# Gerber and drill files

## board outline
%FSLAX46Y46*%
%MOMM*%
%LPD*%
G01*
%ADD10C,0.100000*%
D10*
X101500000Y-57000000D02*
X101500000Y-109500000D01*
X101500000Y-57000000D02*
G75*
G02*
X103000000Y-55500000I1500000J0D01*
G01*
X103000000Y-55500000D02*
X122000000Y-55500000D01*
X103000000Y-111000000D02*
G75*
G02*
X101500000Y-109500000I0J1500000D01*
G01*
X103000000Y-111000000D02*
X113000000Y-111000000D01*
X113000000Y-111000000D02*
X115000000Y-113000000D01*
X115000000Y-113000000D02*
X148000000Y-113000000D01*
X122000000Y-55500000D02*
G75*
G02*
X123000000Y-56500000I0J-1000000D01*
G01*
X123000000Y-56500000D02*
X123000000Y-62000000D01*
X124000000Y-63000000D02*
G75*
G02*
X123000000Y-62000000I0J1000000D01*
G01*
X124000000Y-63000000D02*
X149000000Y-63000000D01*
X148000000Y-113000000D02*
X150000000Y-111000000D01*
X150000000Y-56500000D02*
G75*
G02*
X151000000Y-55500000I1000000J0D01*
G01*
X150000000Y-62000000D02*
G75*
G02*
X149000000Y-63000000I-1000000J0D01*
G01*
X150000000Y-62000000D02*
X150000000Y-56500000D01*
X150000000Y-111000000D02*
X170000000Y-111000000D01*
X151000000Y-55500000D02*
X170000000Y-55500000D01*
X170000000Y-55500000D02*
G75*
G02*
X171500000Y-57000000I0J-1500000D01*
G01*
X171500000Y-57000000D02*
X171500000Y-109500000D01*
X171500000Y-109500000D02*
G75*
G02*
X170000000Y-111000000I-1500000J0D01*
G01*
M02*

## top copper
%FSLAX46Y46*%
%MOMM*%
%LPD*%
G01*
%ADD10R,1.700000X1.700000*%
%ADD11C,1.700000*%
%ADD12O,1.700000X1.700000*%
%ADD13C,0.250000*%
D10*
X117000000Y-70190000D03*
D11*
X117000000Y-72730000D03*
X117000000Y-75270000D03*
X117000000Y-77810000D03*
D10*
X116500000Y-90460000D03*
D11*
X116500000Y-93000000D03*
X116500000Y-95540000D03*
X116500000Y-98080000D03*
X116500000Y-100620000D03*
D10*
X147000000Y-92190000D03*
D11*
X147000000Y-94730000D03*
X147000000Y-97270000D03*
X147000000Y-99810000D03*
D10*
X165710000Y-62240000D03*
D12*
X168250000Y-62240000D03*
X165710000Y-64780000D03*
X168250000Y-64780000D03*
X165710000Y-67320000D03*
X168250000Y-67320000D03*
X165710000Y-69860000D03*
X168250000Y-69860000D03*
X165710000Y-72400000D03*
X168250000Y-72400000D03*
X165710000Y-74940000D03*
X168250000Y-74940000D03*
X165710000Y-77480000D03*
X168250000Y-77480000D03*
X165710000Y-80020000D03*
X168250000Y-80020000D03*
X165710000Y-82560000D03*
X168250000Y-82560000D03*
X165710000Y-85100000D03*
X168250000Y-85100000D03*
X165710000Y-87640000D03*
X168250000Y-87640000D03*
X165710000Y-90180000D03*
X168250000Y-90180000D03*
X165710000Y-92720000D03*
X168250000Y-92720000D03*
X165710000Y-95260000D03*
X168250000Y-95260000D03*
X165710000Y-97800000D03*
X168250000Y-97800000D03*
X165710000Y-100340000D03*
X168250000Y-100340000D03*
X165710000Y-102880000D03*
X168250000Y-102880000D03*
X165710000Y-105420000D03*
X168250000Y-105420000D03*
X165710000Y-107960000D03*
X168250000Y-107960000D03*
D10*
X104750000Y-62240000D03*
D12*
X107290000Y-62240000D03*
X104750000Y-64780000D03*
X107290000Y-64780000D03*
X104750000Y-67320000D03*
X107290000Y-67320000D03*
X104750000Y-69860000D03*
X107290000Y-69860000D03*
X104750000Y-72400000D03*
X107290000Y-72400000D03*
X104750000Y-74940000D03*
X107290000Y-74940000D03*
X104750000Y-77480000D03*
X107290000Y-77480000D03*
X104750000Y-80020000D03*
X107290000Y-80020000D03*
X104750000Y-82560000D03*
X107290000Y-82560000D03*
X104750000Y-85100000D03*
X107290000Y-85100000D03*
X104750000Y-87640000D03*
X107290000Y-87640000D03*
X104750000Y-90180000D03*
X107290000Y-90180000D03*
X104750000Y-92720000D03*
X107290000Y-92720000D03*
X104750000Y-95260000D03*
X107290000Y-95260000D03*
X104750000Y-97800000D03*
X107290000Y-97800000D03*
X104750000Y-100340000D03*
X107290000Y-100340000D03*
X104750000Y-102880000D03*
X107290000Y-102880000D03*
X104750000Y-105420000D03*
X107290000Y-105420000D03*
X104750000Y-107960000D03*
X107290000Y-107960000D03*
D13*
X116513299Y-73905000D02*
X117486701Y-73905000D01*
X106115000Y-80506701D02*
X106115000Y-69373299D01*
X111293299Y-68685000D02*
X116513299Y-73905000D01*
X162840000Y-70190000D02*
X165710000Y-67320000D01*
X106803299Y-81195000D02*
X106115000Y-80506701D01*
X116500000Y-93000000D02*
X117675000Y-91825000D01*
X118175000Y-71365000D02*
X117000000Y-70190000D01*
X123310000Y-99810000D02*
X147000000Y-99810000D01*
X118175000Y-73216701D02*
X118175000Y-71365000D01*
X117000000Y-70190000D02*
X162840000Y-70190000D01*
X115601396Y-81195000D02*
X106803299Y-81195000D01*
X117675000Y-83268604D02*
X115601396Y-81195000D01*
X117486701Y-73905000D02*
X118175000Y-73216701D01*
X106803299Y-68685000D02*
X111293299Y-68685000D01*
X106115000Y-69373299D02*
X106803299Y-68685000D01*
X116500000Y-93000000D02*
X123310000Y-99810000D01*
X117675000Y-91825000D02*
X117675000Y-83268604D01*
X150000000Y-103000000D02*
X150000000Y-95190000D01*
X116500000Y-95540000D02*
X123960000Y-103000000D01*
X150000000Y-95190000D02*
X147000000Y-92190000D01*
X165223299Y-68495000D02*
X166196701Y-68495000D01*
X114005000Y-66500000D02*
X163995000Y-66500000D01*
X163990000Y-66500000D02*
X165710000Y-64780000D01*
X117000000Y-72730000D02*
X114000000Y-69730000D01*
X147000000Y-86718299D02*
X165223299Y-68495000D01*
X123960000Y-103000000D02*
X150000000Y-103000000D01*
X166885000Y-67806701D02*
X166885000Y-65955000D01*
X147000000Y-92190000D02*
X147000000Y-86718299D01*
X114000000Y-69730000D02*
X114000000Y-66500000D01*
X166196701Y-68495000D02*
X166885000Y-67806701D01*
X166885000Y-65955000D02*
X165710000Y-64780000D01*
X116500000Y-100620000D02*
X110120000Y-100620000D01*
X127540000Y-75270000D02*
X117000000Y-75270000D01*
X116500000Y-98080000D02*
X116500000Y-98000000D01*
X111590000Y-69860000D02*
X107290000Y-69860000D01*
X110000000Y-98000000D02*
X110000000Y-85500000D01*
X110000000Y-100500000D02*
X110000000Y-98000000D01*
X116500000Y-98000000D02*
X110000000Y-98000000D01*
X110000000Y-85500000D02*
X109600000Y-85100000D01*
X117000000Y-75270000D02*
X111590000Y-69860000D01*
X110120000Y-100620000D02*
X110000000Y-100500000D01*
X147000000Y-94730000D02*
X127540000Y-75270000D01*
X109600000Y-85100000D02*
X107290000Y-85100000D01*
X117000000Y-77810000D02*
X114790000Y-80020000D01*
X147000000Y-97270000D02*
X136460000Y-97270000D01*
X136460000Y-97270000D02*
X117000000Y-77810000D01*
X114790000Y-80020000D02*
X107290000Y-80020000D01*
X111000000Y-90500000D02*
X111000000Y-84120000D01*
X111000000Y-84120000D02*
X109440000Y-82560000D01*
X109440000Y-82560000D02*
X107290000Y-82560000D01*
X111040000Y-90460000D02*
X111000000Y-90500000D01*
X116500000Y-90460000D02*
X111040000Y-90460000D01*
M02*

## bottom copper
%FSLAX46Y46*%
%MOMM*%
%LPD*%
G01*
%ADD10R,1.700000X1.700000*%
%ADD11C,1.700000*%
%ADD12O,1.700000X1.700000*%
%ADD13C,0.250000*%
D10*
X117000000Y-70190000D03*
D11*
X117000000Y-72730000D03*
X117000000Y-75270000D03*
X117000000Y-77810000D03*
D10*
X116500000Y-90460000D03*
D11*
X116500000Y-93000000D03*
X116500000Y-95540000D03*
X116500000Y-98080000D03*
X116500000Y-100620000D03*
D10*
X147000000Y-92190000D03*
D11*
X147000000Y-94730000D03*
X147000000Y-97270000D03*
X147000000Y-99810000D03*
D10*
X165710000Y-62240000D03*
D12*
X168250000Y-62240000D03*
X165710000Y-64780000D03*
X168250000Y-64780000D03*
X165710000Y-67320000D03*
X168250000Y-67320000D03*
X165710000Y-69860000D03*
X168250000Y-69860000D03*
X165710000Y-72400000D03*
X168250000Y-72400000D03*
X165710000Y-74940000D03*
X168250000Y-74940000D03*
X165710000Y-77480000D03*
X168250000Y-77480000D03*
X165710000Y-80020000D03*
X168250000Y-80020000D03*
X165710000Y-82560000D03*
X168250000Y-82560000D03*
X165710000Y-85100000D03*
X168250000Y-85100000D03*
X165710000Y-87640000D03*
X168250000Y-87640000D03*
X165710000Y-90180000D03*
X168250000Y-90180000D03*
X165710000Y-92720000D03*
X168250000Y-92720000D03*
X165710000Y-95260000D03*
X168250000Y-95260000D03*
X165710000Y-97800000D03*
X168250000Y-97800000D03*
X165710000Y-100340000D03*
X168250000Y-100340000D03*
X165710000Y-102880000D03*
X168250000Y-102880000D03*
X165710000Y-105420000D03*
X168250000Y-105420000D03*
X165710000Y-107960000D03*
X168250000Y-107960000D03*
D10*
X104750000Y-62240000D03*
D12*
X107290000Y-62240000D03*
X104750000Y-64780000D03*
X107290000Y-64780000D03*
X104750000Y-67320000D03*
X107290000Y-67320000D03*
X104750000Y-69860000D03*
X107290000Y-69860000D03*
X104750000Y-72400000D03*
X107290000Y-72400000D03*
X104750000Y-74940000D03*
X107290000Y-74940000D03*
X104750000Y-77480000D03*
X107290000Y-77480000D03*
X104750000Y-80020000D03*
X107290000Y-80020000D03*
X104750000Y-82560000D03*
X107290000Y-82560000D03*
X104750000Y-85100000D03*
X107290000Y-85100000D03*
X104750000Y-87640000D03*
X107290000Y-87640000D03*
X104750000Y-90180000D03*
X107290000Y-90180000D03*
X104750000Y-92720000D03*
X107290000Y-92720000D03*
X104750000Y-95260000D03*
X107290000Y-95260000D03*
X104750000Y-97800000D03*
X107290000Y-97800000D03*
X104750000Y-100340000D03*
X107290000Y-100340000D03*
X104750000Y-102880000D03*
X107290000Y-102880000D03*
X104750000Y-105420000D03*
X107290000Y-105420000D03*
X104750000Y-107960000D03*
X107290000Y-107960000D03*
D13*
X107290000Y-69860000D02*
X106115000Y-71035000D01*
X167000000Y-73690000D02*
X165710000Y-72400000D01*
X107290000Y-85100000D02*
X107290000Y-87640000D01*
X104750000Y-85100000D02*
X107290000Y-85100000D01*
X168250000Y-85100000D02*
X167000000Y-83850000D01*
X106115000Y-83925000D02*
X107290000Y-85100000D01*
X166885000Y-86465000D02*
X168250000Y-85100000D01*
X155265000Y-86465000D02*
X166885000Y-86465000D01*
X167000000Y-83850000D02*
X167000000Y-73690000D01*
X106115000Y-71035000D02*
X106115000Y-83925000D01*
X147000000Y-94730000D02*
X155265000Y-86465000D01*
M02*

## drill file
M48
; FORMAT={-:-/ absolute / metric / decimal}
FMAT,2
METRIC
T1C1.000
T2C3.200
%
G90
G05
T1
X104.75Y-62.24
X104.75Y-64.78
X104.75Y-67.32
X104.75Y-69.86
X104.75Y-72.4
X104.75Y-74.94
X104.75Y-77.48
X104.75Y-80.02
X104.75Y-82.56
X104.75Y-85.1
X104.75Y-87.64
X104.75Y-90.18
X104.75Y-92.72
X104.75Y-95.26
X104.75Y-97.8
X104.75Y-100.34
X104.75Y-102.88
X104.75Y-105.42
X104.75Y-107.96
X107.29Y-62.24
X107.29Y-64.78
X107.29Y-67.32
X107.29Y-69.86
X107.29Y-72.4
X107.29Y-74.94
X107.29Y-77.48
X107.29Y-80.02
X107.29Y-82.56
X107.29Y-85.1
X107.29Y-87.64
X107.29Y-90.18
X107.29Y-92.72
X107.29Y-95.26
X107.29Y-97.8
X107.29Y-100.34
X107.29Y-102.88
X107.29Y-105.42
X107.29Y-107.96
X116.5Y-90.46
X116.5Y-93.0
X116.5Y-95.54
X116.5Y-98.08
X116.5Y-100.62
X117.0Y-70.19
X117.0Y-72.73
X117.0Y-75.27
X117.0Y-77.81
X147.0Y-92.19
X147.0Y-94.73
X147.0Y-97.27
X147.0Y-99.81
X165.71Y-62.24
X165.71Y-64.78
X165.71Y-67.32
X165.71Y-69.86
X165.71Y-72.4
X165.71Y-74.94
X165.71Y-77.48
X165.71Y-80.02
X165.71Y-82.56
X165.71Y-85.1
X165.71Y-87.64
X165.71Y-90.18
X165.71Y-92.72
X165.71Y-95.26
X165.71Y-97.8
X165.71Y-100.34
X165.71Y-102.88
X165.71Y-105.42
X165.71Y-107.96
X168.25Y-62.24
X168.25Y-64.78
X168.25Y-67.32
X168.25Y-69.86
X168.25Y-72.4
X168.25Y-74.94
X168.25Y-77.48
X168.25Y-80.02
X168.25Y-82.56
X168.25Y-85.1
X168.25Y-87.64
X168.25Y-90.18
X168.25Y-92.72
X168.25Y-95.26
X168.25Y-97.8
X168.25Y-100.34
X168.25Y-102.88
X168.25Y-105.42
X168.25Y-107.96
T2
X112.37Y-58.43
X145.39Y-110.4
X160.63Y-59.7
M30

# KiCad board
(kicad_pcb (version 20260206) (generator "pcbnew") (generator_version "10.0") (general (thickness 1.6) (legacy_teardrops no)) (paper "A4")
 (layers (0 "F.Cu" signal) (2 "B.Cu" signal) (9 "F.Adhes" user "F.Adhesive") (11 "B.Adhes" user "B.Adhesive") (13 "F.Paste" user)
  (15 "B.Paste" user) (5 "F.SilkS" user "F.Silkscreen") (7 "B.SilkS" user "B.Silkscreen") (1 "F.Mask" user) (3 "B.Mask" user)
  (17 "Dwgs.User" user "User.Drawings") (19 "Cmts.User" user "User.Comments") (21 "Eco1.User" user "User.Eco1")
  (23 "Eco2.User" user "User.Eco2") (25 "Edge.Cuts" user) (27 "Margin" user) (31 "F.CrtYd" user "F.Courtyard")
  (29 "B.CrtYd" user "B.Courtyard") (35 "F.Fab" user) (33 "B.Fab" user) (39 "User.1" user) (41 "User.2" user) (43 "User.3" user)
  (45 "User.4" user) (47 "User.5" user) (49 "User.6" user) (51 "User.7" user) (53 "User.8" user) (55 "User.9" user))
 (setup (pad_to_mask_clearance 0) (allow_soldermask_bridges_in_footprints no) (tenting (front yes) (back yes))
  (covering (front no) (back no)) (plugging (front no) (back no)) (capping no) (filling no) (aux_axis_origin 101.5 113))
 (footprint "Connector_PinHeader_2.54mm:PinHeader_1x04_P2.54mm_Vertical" (layer "F.Cu") (at 117 70.19)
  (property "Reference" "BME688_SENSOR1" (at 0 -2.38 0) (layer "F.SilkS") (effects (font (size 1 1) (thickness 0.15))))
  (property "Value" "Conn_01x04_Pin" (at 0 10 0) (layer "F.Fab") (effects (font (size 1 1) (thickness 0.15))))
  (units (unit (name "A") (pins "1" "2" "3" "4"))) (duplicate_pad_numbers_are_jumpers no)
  (pad "1" thru_hole rect (at 0 0) (size 1.7 1.7) (drill 1) (layers "*.Cu" "*.Mask") (remove_unused_layers no) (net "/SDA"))
  (pad "2" thru_hole circle (at 0 2.54) (size 1.7 1.7) (drill 1) (layers "*.Cu" "*.Mask") (remove_unused_layers no) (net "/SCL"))
  (pad "3" thru_hole circle (at 0 5.08) (size 1.7 1.7) (drill 1) (layers "*.Cu" "*.Mask") (remove_unused_layers no) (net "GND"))
  (pad "4" thru_hole circle (at 0 7.62) (size 1.7 1.7) (drill 1) (layers "*.Cu" "*.Mask") (remove_unused_layers no) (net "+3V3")))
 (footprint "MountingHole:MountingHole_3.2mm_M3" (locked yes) (layer "F.Cu") (at 160.63 59.7)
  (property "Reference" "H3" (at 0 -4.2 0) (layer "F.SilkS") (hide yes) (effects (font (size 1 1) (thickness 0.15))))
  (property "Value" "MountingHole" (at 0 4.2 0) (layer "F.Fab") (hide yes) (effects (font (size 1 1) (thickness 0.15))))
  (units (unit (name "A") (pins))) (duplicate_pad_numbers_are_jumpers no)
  (pad "" np_thru_hole circle (at 0 0) (size 3.2 3.2) (drill 3.2) (layers "*.Cu" "*.Mask")))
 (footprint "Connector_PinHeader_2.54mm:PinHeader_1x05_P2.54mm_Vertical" (layer "F.Cu") (at 116.5 90.46)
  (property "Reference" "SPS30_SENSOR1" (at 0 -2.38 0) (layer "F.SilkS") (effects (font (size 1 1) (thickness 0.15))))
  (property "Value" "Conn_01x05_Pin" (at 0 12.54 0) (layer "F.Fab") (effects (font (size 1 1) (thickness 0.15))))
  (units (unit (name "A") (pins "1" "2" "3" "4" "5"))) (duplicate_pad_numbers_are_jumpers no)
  (pad "1" thru_hole rect (at 0 0) (size 1.7 1.7) (drill 1) (layers "*.Cu" "*.Mask") (remove_unused_layers no) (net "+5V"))
  (pad "2" thru_hole circle (at 0 2.54) (size 1.7 1.7) (drill 1) (layers "*.Cu" "*.Mask") (remove_unused_layers no) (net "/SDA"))
  (pad "3" thru_hole circle (at 0 5.08) (size 1.7 1.7) (drill 1) (layers "*.Cu" "*.Mask") (remove_unused_layers no) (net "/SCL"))
  (pad "4" thru_hole circle (at 0 7.62) (size 1.7 1.7) (drill 1) (layers "*.Cu" "*.Mask") (remove_unused_layers no) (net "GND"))
  (pad "5" thru_hole circle (at 0 10.16) (size 1.7 1.7) (drill 1) (layers "*.Cu" "*.Mask") (remove_unused_layers no) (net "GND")))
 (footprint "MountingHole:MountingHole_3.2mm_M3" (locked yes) (layer "F.Cu") (at 145.39 110.4)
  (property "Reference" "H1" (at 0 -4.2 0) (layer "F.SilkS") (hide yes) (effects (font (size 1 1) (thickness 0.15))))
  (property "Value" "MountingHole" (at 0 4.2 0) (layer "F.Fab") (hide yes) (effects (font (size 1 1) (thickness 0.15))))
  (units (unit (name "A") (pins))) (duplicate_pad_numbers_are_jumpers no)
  (pad "" np_thru_hole circle (at 0 0) (size 3.2 3.2) (drill 3.2) (layers "*.Cu" "*.Mask")))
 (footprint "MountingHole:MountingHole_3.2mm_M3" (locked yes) (layer "F.Cu") (at 112.37 58.43)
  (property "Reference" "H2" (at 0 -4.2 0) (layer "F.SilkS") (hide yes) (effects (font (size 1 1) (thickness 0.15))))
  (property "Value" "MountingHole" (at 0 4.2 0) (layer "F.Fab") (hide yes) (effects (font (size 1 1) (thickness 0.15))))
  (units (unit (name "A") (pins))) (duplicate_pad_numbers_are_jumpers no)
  (pad "" np_thru_hole circle (at 0 0) (size 3.2 3.2) (drill 3.2) (layers "*.Cu" "*.Mask")))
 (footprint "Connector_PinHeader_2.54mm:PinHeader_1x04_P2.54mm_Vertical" (layer "F.Cu") (at 147 92.19)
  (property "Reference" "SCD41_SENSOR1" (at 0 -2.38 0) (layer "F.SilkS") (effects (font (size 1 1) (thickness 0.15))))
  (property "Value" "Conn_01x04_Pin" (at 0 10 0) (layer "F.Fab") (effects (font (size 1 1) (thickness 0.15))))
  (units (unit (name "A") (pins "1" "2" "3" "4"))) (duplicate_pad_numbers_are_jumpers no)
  (pad "1" thru_hole rect (at 0 0) (size 1.7 1.7) (drill 1) (layers "*.Cu" "*.Mask") (remove_unused_layers no) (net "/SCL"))
  (pad "2" thru_hole circle (at 0 2.54) (size 1.7 1.7) (drill 1) (layers "*.Cu" "*.Mask") (remove_unused_layers no) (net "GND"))
  (pad "3" thru_hole circle (at 0 5.08) (size 1.7 1.7) (drill 1) (layers "*.Cu" "*.Mask") (remove_unused_layers no) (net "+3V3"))
  (pad "4" thru_hole circle (at 0 7.62) (size 1.7 1.7) (drill 1) (layers "*.Cu" "*.Mask") (remove_unused_layers no) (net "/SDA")))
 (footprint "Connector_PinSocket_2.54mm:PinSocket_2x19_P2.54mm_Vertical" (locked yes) (layer "B.Cu") (at 165.71 62.24 180)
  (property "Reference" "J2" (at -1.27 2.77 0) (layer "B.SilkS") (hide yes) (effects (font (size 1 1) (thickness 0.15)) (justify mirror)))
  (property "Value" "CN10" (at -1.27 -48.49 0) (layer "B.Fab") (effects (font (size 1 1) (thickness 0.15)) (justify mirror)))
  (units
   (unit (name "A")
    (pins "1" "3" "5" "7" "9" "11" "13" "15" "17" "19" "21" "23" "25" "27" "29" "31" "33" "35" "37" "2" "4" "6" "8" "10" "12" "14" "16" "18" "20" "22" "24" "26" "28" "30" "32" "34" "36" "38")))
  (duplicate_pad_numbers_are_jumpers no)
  (pad "1" thru_hole rect (at 0 0 180) (size 1.7 1.7) (drill 1) (layers "*.Cu" "*.Mask") (remove_unused_layers no)
   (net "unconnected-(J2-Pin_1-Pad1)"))
  (pad "2" thru_hole oval (at -2.54 0 180) (size 1.7 1.7) (drill 1) (layers "*.Cu" "*.Mask") (remove_unused_layers no)
   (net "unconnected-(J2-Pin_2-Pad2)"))
  (pad "3" thru_hole oval (at 0 -2.54 180) (size 1.7 1.7) (drill 1) (layers "*.Cu" "*.Mask") (remove_unused_layers no) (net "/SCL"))
  (pad "4" thru_hole oval (at -2.54 -2.54 180) (size 1.7 1.7) (drill 1) (layers "*.Cu" "*.Mask") (remove_unused_layers no)
   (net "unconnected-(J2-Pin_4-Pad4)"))
  (pad "5" thru_hole oval (at 0 -5.08 180) (size 1.7 1.7) (drill 1) (layers "*.Cu" "*.Mask") (remove_unused_layers no) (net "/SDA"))
  (pad "6" thru_hole oval (at -2.54 -5.08 180) (size 1.7 1.7) (drill 1) (layers "*.Cu" "*.Mask") (remove_unused_layers no)
   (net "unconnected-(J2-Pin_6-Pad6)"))
  (pad "7" thru_hole oval (at 0 -7.62 180) (size 1.7 1.7) (drill 1) (layers "*.Cu" "*.Mask") (remove_unused_layers no) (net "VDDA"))
  (pad "8" thru_hole oval (at -2.54 -7.62 180) (size 1.7 1.7) (drill 1) (layers "*.Cu" "*.Mask") (remove_unused_layers no)
   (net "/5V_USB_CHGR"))
  (pad "9" thru_hole oval (at 0 -10.16 180) (size 1.7 1.7) (drill 1) (layers "*.Cu" "*.Mask") (remove_unused_layers no) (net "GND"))
  (pad "10" thru_hole oval (at -2.54 -10.16 180) (size 1.7 1.7) (drill 1) (layers "*.Cu" "*.Mask") (remove_unused_layers no)
   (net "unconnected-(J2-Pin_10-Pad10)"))
  (pad "11" thru_hole oval (at 0 -12.7 180) (size 1.7 1.7) (drill 1) (layers "*.Cu" "*.Mask") (remove_unused_layers no)
   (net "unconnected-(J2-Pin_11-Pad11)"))
  (pad "12" thru_hole oval (at -2.54 -12.7 180) (size 1.7 1.7) (drill 1) (layers "*.Cu" "*.Mask") (remove_unused_layers no)
   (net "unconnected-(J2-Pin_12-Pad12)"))
  (pad "13" thru_hole oval (at 0 -15.24 180) (size 1.7 1.7) (drill 1) (layers "*.Cu" "*.Mask") (remove_unused_layers no)
   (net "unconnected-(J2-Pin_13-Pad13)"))
  (pad "14" thru_hole oval (at -2.54 -15.24 180) (size 1.7 1.7) (drill 1) (layers "*.Cu" "*.Mask") (remove_unused_layers no)
   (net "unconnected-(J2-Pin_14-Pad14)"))
  (pad "15" thru_hole oval (at 0 -17.78 180) (size 1.7 1.7) (drill 1) (layers "*.Cu" "*.Mask") (remove_unused_layers no)
   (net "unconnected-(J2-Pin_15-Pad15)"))
  (pad "16" thru_hole oval (at -2.54 -17.78 180) (size 1.7 1.7) (drill 1) (layers "*.Cu" "*.Mask") (remove_unused_layers no)
   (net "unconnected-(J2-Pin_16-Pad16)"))
  (pad "17" thru_hole oval (at 0 -20.32 180) (size 1.7 1.7) (drill 1) (layers "*.Cu" "*.Mask") (remove_unused_layers no)
   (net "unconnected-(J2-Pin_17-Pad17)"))
  (pad "18" thru_hole oval (at -2.54 -20.32 180) (size 1.7 1.7) (drill 1) (layers "*.Cu" "*.Mask") (remove_unused_layers no)
   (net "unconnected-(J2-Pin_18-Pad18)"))
  (pad "19" thru_hole oval (at 0 -22.86 180) (size 1.7 1.7) (drill 1) (layers "*.Cu" "*.Mask") (remove_unused_layers no)
   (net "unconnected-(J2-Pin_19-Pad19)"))
  (pad "20" thru_hole oval (at -2.54 -22.86 180) (size 1.7 1.7) (drill 1) (layers "*.Cu" "*.Mask") (remove_unused_layers no) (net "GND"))
  (pad "21" thru_hole oval (at 0 -25.4 180) (size 1.7 1.7) (drill 1) (layers "*.Cu" "*.Mask") (remove_unused_layers no)
   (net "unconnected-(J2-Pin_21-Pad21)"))
  (pad "22" thru_hole oval (at -2.54 -25.4 180) (size 1.7 1.7) (drill 1) (layers "*.Cu" "*.Mask") (remove_unused_layers no)
   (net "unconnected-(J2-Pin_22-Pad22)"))
  (pad "23" thru_hole oval (at 0 -27.94 180) (size 1.7 1.7) (drill 1) (layers "*.Cu" "*.Mask") (remove_unused_layers no)
   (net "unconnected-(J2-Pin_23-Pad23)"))
  (pad "24" thru_hole oval (at -2.54 -27.94 180) (size 1.7 1.7) (drill 1) (layers "*.Cu" "*.Mask") (remove_unused_layers no)
   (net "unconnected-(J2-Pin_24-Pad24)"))
  (pad "25" thru_hole oval (at 0 -30.48 180) (size 1.7 1.7) (drill 1) (layers "*.Cu" "*.Mask") (remove_unused_layers no)
   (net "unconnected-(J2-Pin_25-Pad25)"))
  (pad "26" thru_hole oval (at -2.54 -30.48 180) (size 1.7 1.7) (drill 1) (layers "*.Cu" "*.Mask") (remove_unused_layers no)
   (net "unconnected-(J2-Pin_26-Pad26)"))
  (pad "27" thru_hole oval (at 0 -33.02 180) (size 1.7 1.7) (drill 1) (layers "*.Cu" "*.Mask") (remove_unused_layers no)
   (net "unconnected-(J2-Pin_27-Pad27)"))
  (pad "28" thru_hole oval (at -2.54 -33.02 180) (size 1.7 1.7) (drill 1) (layers "*.Cu" "*.Mask") (remove_unused_layers no)
   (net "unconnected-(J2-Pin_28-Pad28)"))
  (pad "29" thru_hole oval (at 0 -35.56 180) (size 1.7 1.7) (drill 1) (layers "*.Cu" "*.Mask") (remove_unused_layers no)
   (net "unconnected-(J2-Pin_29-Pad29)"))
  (pad "30" thru_hole oval (at -2.54 -35.56 180) (size 1.7 1.7) (drill 1) (layers "*.Cu" "*.Mask") (remove_unused_layers no)
   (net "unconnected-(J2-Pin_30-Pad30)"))
  (pad "31" thru_hole oval (at 0 -38.1 180) (size 1.7 1.7) (drill 1) (layers "*.Cu" "*.Mask") (remove_unused_layers no)
   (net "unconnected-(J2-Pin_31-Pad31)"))
  (pad "32" thru_hole oval (at -2.54 -38.1 180) (size 1.7 1.7) (drill 1) (layers "*.Cu" "*.Mask") (remove_unused_layers no) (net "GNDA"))
  (pad "33" thru_hole oval (at 0 -40.64 180) (size 1.7 1.7) (drill 1) (layers "*.Cu" "*.Mask") (remove_unused_layers no)
   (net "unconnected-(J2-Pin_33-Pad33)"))
  (pad "34" thru_hole oval (at -2.54 -40.64 180) (size 1.7 1.7) (drill 1) (layers "*.Cu" "*.Mask") (remove_unused_layers no)
   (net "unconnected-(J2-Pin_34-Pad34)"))
  (pad "35" thru_hole oval (at 0 -43.18 180) (size 1.7 1.7) (drill 1) (layers "*.Cu" "*.Mask") (remove_unused_layers no)
   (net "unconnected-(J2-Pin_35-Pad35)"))
  (pad "36" thru_hole oval (at -2.54 -43.18 180) (size 1.7 1.7) (drill 1) (layers "*.Cu" "*.Mask") (remove_unused_layers no)
   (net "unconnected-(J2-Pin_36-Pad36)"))
  (pad "37" thru_hole oval (at 0 -45.72 180) (size 1.7 1.7) (drill 1) (layers "*.Cu" "*.Mask") (remove_unused_layers no)
   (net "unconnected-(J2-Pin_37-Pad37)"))
  (pad "38" thru_hole oval (at -2.54 -45.72 180) (size 1.7 1.7) (drill 1) (layers "*.Cu" "*.Mask") (remove_unused_layers no)
   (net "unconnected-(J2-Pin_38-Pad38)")))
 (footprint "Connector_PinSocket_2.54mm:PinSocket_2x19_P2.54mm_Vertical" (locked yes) (layer "B.Cu") (at 104.75 62.24 180)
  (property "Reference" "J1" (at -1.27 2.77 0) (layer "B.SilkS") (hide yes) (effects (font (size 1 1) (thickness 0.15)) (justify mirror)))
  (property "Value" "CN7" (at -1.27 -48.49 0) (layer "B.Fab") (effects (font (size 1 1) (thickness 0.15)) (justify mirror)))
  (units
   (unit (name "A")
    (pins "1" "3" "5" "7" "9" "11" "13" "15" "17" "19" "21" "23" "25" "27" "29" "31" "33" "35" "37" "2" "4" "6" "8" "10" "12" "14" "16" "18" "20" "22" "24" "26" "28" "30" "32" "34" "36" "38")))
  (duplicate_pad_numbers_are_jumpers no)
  (pad "1" thru_hole rect (at 0 0 180) (size 1.7 1.7) (drill 1) (layers "*.Cu" "*.Mask") (remove_unused_layers no)
   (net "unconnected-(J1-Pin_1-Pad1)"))
  (pad "2" thru_hole oval (at -2.54 0 180) (size 1.7 1.7) (drill 1) (layers "*.Cu" "*.Mask") (remove_unused_layers no)
   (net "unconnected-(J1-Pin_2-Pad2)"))
  (pad "3" thru_hole oval (at 0 -2.54 180) (size 1.7 1.7) (drill 1) (layers "*.Cu" "*.Mask") (remove_unused_layers no)
   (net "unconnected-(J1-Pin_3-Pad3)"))
  (pad "4" thru_hole oval (at -2.54 -2.54 180) (size 1.7 1.7) (drill 1) (layers "*.Cu" "*.Mask") (remove_unused_layers no)
   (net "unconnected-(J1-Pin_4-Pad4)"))
  (pad "5" thru_hole oval (at 0 -5.08 180) (size 1.7 1.7) (drill 1) (layers "*.Cu" "*.Mask") (remove_unused_layers no) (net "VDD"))
  (pad "6" thru_hole oval (at -2.54 -5.08 180) (size 1.7 1.7) (drill 1) (layers "*.Cu" "*.Mask") (remove_unused_layers no) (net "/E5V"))
  (pad "7" thru_hole oval (at 0 -7.62 180) (size 1.7 1.7) (drill 1) (layers "*.Cu" "*.Mask") (remove_unused_layers no)
   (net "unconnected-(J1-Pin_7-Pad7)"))
  (pad "8" thru_hole oval (at -2.54 -7.62 180) (size 1.7 1.7) (drill 1) (layers "*.Cu" "*.Mask") (remove_unused_layers no) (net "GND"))
  (pad "9" thru_hole oval (at 0 -10.16 180) (size 1.7 1.7) (drill 1) (layers "*.Cu" "*.Mask") (remove_unused_layers no)
   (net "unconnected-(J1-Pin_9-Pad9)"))
  (pad "10" thru_hole oval (at -2.54 -10.16 180) (size 1.7 1.7) (drill 1) (layers "*.Cu" "*.Mask") (remove_unused_layers no)
   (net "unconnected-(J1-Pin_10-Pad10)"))
  (pad "11" thru_hole oval (at 0 -12.7 180) (size 1.7 1.7) (drill 1) (layers "*.Cu" "*.Mask") (remove_unused_layers no)
   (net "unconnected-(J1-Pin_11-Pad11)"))
  (pad "12" thru_hole oval (at -2.54 -12.7 180) (size 1.7 1.7) (drill 1) (layers "*.Cu" "*.Mask") (remove_unused_layers no) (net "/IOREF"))
  (pad "13" thru_hole oval (at 0 -15.24 180) (size 1.7 1.7) (drill 1) (layers "*.Cu" "*.Mask") (remove_unused_layers no)
   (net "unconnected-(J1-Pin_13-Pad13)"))
  (pad "14" thru_hole oval (at -2.54 -15.24 180) (size 1.7 1.7) (drill 1) (layers "*.Cu" "*.Mask") (remove_unused_layers no) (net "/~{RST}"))
  (pad "15" thru_hole oval (at 0 -17.78 180) (size 1.7 1.7) (drill 1) (layers "*.Cu" "*.Mask") (remove_unused_layers no)
   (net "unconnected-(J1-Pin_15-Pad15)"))
  (pad "16" thru_hole oval (at -2.54 -17.78 180) (size 1.7 1.7) (drill 1) (layers "*.Cu" "*.Mask") (remove_unused_layers no) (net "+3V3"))
  (pad "17" thru_hole oval (at 0 -20.32 180) (size 1.7 1.7) (drill 1) (layers "*.Cu" "*.Mask") (remove_unused_layers no)
   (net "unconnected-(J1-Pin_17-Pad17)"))
  (pad "18" thru_hole oval (at -2.54 -20.32 180) (size 1.7 1.7) (drill 1) (layers "*.Cu" "*.Mask") (remove_unused_layers no) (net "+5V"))
  (pad "19" thru_hole oval (at 0 -22.86 180) (size 1.7 1.7) (drill 1) (layers "*.Cu" "*.Mask") (remove_unused_layers no) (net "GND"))
  (pad "20" thru_hole oval (at -2.54 -22.86 180) (size 1.7 1.7) (drill 1) (layers "*.Cu" "*.Mask") (remove_unused_layers no) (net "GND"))
  (pad "21" thru_hole oval (at 0 -25.4 180) (size 1.7 1.7) (drill 1) (layers "*.Cu" "*.Mask") (remove_unused_layers no)
   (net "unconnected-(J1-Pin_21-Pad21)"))
  (pad "22" thru_hole oval (at -2.54 -25.4 180) (size 1.7 1.7) (drill 1) (layers "*.Cu" "*.Mask") (remove_unused_layers no) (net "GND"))
  (pad "23" thru_hole oval (at 0 -27.94 180) (size 1.7 1.7) (drill 1) (layers "*.Cu" "*.Mask") (remove_unused_layers no)
   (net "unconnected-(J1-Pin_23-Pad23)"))
  (pad "24" thru_hole oval (at -2.54 -27.94 180) (size 1.7 1.7) (drill 1) (layers "*.Cu" "*.Mask") (remove_unused_layers no) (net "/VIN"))
  (pad "25" thru_hole oval (at 0 -30.48 180) (size 1.7 1.7) (drill 1) (layers "*.Cu" "*.Mask") (remove_unused_layers no)
   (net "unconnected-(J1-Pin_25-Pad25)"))
  (pad "26" thru_hole oval (at -2.54 -30.48 180) (size 1.7 1.7) (drill 1) (layers "*.Cu" "*.Mask") (remove_unused_layers no)
   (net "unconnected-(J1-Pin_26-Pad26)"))
  (pad "27" thru_hole oval (at 0 -33.02 180) (size 1.7 1.7) (drill 1) (layers "*.Cu" "*.Mask") (remove_unused_layers no)
   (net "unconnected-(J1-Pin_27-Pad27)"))
  (pad "28" thru_hole oval (at -2.54 -33.02 180) (size 1.7 1.7) (drill 1) (layers "*.Cu" "*.Mask") (remove_unused_layers no)
   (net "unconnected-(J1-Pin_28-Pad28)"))
  (pad "29" thru_hole oval (at 0 -35.56 180) (size 1.7 1.7) (drill 1) (layers "*.Cu" "*.Mask") (remove_unused_layers no)
   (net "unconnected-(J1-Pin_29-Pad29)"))
  (pad "30" thru_hole oval (at -2.54 -35.56 180) (size 1.7 1.7) (drill 1) (layers "*.Cu" "*.Mask") (remove_unused_layers no)
   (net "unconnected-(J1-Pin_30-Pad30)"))
  (pad "31" thru_hole oval (at 0 -38.1 180) (size 1.7 1.7) (drill 1) (layers "*.Cu" "*.Mask") (remove_unused_layers no)
   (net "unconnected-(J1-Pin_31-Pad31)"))
  (pad "32" thru_hole oval (at -2.54 -38.1 180) (size 1.7 1.7) (drill 1) (layers "*.Cu" "*.Mask") (remove_unused_layers no)
   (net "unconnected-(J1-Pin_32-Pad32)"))
  (pad "33" thru_hole oval (at 0 -40.64 180) (size 1.7 1.7) (drill 1) (layers "*.Cu" "*.Mask") (remove_unused_layers no) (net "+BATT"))
  (pad "34" thru_hole oval (at -2.54 -40.64 180) (size 1.7 1.7) (drill 1) (layers "*.Cu" "*.Mask") (remove_unused_layers no)
   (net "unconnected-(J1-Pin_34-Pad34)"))
  (pad "35" thru_hole oval (at 0 -43.18 180) (size 1.7 1.7) (drill 1) (layers "*.Cu" "*.Mask") (remove_unused_layers no)
   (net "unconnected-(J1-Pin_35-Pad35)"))
  (pad "36" thru_hole oval (at -2.54 -43.18 180) (size 1.7 1.7) (drill 1) (layers "*.Cu" "*.Mask") (remove_unused_layers no)
   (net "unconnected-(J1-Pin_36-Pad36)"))
  (pad "37" thru_hole oval (at 0 -45.72 180) (size 1.7 1.7) (drill 1) (layers "*.Cu" "*.Mask") (remove_unused_layers no)
   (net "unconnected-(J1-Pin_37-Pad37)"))
  (pad "38" thru_hole oval (at -2.54 -45.72 180) (size 1.7 1.7) (drill 1) (layers "*.Cu" "*.Mask") (remove_unused_layers no)
   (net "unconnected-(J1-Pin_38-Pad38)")))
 (gr_line (start 101.5 57) (end 101.5 109.5) (stroke (width 0.1) (type solid)) (layer "Edge.Cuts"))
 (gr_arc (start 101.5 57) (mid 101.93934 55.93934) (end 103 55.5) (stroke (width 0.1) (type solid)) (layer "Edge.Cuts"))
 (gr_line (start 103 55.5) (end 122 55.5) (stroke (width 0.1) (type solid)) (layer "Edge.Cuts"))
 (gr_arc (start 103 111) (mid 101.93934 110.56066) (end 101.5 109.5) (stroke (width 0.1) (type solid)) (layer "Edge.Cuts"))
 (gr_line (start 103 111) (end 113 111) (stroke (width 0.1) (type solid)) (layer "Edge.Cuts"))
 (gr_line (start 113 111) (end 115 113) (stroke (width 0.1) (type solid)) (layer "Edge.Cuts"))
 (gr_line (start 115 113) (end 148 113) (stroke (width 0.1) (type solid)) (layer "Edge.Cuts"))
 (gr_arc (start 122 55.5) (mid 122.707107 55.792893) (end 123 56.5) (stroke (width 0.1) (type solid)) (layer "Edge.Cuts"))
 (gr_line (start 123 56.5) (end 123 62) (stroke (width 0.1) (type solid)) (layer "Edge.Cuts"))
 (gr_arc (start 124 63) (mid 123.292893 62.707107) (end 123 62) (stroke (width 0.1) (type solid)) (layer "Edge.Cuts"))
 (gr_line (start 124 63) (end 149 63) (stroke (width 0.1) (type solid)) (layer "Edge.Cuts"))
 (gr_line (start 148 113) (end 150 111) (stroke (width 0.1) (type solid)) (layer "Edge.Cuts"))
 (gr_arc (start 150 56.5) (mid 150.292893 55.792893) (end 151 55.5) (stroke (width 0.1) (type solid)) (layer "Edge.Cuts"))
 (gr_arc (start 150 62) (mid 149.707107 62.707107) (end 149 63) (stroke (width 0.1) (type solid)) (layer "Edge.Cuts"))
 (gr_line (start 150 62) (end 150 56.5) (stroke (width 0.1) (type solid)) (layer "Edge.Cuts"))
 (gr_line (start 150 111) (end 170 111) (stroke (width 0.1) (type solid)) (layer "Edge.Cuts"))
 (gr_line (start 151 55.5) (end 170 55.5) (stroke (width 0.1) (type solid)) (layer "Edge.Cuts"))
 (gr_arc (start 170 55.5) (mid 171.06066 55.93934) (end 171.5 57) (stroke (width 0.1) (type solid)) (layer "Edge.Cuts"))
 (gr_line (start 171.5 57) (end 171.5 109.5) (stroke (width 0.1) (type solid)) (layer "Edge.Cuts"))
 (gr_arc (start 171.5 109.5) (mid 171.06066 110.56066) (end 170 111) (stroke (width 0.1) (type solid)) (layer "Edge.Cuts"))
 (segment (start 116.513299 73.905) (end 117.486701 73.905) (width 0.25) (layer "F.Cu") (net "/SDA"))
 (segment (start 106.115 80.506701) (end 106.115 69.373299) (width 0.25) (layer "F.Cu") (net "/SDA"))
 (segment (start 111.293299 68.685) (end 116.513299 73.905) (width 0.25) (layer "F.Cu") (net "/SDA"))
 (segment (start 162.84 70.19) (end 165.71 67.32) (width 0.25) (layer "F.Cu") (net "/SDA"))
 (segment (start 106.803299 81.195) (end 106.115 80.506701) (width 0.25) (layer "F.Cu") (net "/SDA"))
 (segment (start 116.5 93) (end 117.675 91.825) (width 0.25) (layer "F.Cu") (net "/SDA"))
 (segment (start 118.175 71.365) (end 117 70.19) (width 0.25) (layer "F.Cu") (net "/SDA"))
 (segment (start 123.31 99.81) (end 147 99.81) (width 0.25) (layer "F.Cu") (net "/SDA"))
 (segment (start 118.175 73.216701) (end 118.175 71.365) (width 0.25) (layer "F.Cu") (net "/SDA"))
 (segment (start 117 70.19) (end 162.84 70.19) (width 0.25) (layer "F.Cu") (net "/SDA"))
 (segment (start 115.601396 81.195) (end 106.803299 81.195) (width 0.25) (layer "F.Cu") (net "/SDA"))
 (segment (start 117.675 83.268604) (end 115.601396 81.195) (width 0.25) (layer "F.Cu") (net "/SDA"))
 (segment (start 117.486701 73.905) (end 118.175 73.216701) (width 0.25) (layer "F.Cu") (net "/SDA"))
 (segment (start 106.803299 68.685) (end 111.293299 68.685) (width 0.25) (layer "F.Cu") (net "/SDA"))
 (segment (start 106.115 69.373299) (end 106.803299 68.685) (width 0.25) (layer "F.Cu") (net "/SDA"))
 (segment (start 116.5 93) (end 123.31 99.81) (width 0.25) (layer "F.Cu") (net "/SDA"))
 (segment (start 117.675 91.825) (end 117.675 83.268604) (width 0.25) (layer "F.Cu") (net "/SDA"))
 (segment (start 150 103) (end 150 95.19) (width 0.25) (layer "F.Cu") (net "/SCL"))
 (segment (start 116.5 95.54) (end 123.96 103) (width 0.25) (layer "F.Cu") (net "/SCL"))
 (segment (start 150 95.19) (end 147 92.19) (width 0.25) (layer "F.Cu") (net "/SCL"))
 (segment (start 165.223299 68.495) (end 166.196701 68.495) (width 0.25) (layer "F.Cu") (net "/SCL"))
 (segment (start 114.005 66.5) (end 163.995 66.5) (width 0.25) (layer "F.Cu") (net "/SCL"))
 (segment (start 163.99 66.5) (end 165.71 64.78) (width 0.25) (layer "F.Cu") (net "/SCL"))
 (segment (start 117 72.73) (end 114 69.73) (width 0.25) (layer "F.Cu") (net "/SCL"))
 (segment (start 147 86.718299) (end 165.223299 68.495) (width 0.25) (layer "F.Cu") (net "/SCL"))
 (segment (start 123.96 103) (end 150 103) (width 0.25) (layer "F.Cu") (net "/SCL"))
 (segment (start 166.885 67.806701) (end 166.885 65.955) (width 0.25) (layer "F.Cu") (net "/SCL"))
 (segment (start 147 92.19) (end 147 86.718299) (width 0.25) (layer "F.Cu") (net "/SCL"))
 (segment (start 114 69.73) (end 114 66.5) (width 0.25) (layer "F.Cu") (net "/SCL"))
 (segment (start 166.196701 68.495) (end 166.885 67.806701) (width 0.25) (layer "F.Cu") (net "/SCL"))
 (segment (start 166.885 65.955) (end 165.71 64.78) (width 0.25) (layer "F.Cu") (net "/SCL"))
 (segment (start 116.5 100.62) (end 110.12 100.62) (width 0.25) (layer "F.Cu") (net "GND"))
 (segment (start 127.54 75.27) (end 117 75.27) (width 0.25) (layer "F.Cu") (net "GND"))
 (segment (start 116.5 98.08) (end 116.5 98) (width 0.25) (layer "F.Cu") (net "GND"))
 (segment (start 111.59 69.86) (end 107.29 69.86) (width 0.25) (layer "F.Cu") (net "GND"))
 (segment (start 110 98) (end 110 85.5) (width 0.25) (layer "F.Cu") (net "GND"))
 (segment (start 110 100.5) (end 110 98) (width 0.25) (layer "F.Cu") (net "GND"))
 (segment (start 116.5 98) (end 110 98) (width 0.25) (layer "F.Cu") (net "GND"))
 (segment (start 110 85.5) (end 109.6 85.1) (width 0.25) (layer "F.Cu") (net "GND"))
 (segment (start 117 75.27) (end 111.59 69.86) (width 0.25) (layer "F.Cu") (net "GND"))
 (segment (start 110.12 100.62) (end 110 100.5) (width 0.25) (layer "F.Cu") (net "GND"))
 (segment (start 147 94.73) (end 127.54 75.27) (width 0.25) (layer "F.Cu") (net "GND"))
 (segment (start 109.6 85.1) (end 107.29 85.1) (width 0.25) (layer "F.Cu") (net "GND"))
 (segment (start 107.29 69.86) (end 106.115 71.035) (width 0.25) (layer "B.Cu") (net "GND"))
 (segment (start 167 73.69) (end 165.71 72.4) (width 0.25) (layer "B.Cu") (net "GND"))
 (segment (start 107.29 85.1) (end 107.29 87.64) (width 0.25) (layer "B.Cu") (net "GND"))
 (segment (start 104.75 85.1) (end 107.29 85.1) (width 0.25) (layer "B.Cu") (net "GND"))
 (segment (start 168.25 85.1) (end 167 83.85) (width 0.25) (layer "B.Cu") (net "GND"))
 (segment (start 106.115 83.925) (end 107.29 85.1) (width 0.25) (layer "B.Cu") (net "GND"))
 (segment (start 166.885 86.465) (end 168.25 85.1) (width 0.25) (layer "B.Cu") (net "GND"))
 (segment (start 155.265 86.465) (end 166.885 86.465) (width 0.25) (layer "B.Cu") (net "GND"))
 (segment (start 167 83.85) (end 167 73.69) (width 0.25) (layer "B.Cu") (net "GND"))
 (segment (start 106.115 71.035) (end 106.115 83.925) (width 0.25) (layer "B.Cu") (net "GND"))
 (segment (start 147 94.73) (end 155.265 86.465) (width 0.25) (layer "B.Cu") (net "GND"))
 (segment (start 117 77.81) (end 114.79 80.02) (width 0.25) (layer "F.Cu") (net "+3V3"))
 (segment (start 147 97.27) (end 136.46 97.27) (width 0.25) (layer "F.Cu") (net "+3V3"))
 (segment (start 136.46 97.27) (end 117 77.81) (width 0.25) (layer "F.Cu") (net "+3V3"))
 (segment (start 114.79 80.02) (end 107.29 80.02) (width 0.25) (layer "F.Cu") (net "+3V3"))
 (segment (start 111 90.5) (end 111 84.12) (width 0.25) (layer "F.Cu") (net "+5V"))
 (segment (start 111 84.12) (end 109.44 82.56) (width 0.25) (layer "F.Cu") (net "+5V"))
 (segment (start 109.44 82.56) (end 107.29 82.56) (width 0.25) (layer "F.Cu") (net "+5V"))
 (segment (start 111.04 90.46) (end 111 90.5) (width 0.25) (layer "F.Cu") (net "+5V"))
 (segment (start 116.5 90.46) (end 111.04 90.46) (width 0.25) (layer "F.Cu") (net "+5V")))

